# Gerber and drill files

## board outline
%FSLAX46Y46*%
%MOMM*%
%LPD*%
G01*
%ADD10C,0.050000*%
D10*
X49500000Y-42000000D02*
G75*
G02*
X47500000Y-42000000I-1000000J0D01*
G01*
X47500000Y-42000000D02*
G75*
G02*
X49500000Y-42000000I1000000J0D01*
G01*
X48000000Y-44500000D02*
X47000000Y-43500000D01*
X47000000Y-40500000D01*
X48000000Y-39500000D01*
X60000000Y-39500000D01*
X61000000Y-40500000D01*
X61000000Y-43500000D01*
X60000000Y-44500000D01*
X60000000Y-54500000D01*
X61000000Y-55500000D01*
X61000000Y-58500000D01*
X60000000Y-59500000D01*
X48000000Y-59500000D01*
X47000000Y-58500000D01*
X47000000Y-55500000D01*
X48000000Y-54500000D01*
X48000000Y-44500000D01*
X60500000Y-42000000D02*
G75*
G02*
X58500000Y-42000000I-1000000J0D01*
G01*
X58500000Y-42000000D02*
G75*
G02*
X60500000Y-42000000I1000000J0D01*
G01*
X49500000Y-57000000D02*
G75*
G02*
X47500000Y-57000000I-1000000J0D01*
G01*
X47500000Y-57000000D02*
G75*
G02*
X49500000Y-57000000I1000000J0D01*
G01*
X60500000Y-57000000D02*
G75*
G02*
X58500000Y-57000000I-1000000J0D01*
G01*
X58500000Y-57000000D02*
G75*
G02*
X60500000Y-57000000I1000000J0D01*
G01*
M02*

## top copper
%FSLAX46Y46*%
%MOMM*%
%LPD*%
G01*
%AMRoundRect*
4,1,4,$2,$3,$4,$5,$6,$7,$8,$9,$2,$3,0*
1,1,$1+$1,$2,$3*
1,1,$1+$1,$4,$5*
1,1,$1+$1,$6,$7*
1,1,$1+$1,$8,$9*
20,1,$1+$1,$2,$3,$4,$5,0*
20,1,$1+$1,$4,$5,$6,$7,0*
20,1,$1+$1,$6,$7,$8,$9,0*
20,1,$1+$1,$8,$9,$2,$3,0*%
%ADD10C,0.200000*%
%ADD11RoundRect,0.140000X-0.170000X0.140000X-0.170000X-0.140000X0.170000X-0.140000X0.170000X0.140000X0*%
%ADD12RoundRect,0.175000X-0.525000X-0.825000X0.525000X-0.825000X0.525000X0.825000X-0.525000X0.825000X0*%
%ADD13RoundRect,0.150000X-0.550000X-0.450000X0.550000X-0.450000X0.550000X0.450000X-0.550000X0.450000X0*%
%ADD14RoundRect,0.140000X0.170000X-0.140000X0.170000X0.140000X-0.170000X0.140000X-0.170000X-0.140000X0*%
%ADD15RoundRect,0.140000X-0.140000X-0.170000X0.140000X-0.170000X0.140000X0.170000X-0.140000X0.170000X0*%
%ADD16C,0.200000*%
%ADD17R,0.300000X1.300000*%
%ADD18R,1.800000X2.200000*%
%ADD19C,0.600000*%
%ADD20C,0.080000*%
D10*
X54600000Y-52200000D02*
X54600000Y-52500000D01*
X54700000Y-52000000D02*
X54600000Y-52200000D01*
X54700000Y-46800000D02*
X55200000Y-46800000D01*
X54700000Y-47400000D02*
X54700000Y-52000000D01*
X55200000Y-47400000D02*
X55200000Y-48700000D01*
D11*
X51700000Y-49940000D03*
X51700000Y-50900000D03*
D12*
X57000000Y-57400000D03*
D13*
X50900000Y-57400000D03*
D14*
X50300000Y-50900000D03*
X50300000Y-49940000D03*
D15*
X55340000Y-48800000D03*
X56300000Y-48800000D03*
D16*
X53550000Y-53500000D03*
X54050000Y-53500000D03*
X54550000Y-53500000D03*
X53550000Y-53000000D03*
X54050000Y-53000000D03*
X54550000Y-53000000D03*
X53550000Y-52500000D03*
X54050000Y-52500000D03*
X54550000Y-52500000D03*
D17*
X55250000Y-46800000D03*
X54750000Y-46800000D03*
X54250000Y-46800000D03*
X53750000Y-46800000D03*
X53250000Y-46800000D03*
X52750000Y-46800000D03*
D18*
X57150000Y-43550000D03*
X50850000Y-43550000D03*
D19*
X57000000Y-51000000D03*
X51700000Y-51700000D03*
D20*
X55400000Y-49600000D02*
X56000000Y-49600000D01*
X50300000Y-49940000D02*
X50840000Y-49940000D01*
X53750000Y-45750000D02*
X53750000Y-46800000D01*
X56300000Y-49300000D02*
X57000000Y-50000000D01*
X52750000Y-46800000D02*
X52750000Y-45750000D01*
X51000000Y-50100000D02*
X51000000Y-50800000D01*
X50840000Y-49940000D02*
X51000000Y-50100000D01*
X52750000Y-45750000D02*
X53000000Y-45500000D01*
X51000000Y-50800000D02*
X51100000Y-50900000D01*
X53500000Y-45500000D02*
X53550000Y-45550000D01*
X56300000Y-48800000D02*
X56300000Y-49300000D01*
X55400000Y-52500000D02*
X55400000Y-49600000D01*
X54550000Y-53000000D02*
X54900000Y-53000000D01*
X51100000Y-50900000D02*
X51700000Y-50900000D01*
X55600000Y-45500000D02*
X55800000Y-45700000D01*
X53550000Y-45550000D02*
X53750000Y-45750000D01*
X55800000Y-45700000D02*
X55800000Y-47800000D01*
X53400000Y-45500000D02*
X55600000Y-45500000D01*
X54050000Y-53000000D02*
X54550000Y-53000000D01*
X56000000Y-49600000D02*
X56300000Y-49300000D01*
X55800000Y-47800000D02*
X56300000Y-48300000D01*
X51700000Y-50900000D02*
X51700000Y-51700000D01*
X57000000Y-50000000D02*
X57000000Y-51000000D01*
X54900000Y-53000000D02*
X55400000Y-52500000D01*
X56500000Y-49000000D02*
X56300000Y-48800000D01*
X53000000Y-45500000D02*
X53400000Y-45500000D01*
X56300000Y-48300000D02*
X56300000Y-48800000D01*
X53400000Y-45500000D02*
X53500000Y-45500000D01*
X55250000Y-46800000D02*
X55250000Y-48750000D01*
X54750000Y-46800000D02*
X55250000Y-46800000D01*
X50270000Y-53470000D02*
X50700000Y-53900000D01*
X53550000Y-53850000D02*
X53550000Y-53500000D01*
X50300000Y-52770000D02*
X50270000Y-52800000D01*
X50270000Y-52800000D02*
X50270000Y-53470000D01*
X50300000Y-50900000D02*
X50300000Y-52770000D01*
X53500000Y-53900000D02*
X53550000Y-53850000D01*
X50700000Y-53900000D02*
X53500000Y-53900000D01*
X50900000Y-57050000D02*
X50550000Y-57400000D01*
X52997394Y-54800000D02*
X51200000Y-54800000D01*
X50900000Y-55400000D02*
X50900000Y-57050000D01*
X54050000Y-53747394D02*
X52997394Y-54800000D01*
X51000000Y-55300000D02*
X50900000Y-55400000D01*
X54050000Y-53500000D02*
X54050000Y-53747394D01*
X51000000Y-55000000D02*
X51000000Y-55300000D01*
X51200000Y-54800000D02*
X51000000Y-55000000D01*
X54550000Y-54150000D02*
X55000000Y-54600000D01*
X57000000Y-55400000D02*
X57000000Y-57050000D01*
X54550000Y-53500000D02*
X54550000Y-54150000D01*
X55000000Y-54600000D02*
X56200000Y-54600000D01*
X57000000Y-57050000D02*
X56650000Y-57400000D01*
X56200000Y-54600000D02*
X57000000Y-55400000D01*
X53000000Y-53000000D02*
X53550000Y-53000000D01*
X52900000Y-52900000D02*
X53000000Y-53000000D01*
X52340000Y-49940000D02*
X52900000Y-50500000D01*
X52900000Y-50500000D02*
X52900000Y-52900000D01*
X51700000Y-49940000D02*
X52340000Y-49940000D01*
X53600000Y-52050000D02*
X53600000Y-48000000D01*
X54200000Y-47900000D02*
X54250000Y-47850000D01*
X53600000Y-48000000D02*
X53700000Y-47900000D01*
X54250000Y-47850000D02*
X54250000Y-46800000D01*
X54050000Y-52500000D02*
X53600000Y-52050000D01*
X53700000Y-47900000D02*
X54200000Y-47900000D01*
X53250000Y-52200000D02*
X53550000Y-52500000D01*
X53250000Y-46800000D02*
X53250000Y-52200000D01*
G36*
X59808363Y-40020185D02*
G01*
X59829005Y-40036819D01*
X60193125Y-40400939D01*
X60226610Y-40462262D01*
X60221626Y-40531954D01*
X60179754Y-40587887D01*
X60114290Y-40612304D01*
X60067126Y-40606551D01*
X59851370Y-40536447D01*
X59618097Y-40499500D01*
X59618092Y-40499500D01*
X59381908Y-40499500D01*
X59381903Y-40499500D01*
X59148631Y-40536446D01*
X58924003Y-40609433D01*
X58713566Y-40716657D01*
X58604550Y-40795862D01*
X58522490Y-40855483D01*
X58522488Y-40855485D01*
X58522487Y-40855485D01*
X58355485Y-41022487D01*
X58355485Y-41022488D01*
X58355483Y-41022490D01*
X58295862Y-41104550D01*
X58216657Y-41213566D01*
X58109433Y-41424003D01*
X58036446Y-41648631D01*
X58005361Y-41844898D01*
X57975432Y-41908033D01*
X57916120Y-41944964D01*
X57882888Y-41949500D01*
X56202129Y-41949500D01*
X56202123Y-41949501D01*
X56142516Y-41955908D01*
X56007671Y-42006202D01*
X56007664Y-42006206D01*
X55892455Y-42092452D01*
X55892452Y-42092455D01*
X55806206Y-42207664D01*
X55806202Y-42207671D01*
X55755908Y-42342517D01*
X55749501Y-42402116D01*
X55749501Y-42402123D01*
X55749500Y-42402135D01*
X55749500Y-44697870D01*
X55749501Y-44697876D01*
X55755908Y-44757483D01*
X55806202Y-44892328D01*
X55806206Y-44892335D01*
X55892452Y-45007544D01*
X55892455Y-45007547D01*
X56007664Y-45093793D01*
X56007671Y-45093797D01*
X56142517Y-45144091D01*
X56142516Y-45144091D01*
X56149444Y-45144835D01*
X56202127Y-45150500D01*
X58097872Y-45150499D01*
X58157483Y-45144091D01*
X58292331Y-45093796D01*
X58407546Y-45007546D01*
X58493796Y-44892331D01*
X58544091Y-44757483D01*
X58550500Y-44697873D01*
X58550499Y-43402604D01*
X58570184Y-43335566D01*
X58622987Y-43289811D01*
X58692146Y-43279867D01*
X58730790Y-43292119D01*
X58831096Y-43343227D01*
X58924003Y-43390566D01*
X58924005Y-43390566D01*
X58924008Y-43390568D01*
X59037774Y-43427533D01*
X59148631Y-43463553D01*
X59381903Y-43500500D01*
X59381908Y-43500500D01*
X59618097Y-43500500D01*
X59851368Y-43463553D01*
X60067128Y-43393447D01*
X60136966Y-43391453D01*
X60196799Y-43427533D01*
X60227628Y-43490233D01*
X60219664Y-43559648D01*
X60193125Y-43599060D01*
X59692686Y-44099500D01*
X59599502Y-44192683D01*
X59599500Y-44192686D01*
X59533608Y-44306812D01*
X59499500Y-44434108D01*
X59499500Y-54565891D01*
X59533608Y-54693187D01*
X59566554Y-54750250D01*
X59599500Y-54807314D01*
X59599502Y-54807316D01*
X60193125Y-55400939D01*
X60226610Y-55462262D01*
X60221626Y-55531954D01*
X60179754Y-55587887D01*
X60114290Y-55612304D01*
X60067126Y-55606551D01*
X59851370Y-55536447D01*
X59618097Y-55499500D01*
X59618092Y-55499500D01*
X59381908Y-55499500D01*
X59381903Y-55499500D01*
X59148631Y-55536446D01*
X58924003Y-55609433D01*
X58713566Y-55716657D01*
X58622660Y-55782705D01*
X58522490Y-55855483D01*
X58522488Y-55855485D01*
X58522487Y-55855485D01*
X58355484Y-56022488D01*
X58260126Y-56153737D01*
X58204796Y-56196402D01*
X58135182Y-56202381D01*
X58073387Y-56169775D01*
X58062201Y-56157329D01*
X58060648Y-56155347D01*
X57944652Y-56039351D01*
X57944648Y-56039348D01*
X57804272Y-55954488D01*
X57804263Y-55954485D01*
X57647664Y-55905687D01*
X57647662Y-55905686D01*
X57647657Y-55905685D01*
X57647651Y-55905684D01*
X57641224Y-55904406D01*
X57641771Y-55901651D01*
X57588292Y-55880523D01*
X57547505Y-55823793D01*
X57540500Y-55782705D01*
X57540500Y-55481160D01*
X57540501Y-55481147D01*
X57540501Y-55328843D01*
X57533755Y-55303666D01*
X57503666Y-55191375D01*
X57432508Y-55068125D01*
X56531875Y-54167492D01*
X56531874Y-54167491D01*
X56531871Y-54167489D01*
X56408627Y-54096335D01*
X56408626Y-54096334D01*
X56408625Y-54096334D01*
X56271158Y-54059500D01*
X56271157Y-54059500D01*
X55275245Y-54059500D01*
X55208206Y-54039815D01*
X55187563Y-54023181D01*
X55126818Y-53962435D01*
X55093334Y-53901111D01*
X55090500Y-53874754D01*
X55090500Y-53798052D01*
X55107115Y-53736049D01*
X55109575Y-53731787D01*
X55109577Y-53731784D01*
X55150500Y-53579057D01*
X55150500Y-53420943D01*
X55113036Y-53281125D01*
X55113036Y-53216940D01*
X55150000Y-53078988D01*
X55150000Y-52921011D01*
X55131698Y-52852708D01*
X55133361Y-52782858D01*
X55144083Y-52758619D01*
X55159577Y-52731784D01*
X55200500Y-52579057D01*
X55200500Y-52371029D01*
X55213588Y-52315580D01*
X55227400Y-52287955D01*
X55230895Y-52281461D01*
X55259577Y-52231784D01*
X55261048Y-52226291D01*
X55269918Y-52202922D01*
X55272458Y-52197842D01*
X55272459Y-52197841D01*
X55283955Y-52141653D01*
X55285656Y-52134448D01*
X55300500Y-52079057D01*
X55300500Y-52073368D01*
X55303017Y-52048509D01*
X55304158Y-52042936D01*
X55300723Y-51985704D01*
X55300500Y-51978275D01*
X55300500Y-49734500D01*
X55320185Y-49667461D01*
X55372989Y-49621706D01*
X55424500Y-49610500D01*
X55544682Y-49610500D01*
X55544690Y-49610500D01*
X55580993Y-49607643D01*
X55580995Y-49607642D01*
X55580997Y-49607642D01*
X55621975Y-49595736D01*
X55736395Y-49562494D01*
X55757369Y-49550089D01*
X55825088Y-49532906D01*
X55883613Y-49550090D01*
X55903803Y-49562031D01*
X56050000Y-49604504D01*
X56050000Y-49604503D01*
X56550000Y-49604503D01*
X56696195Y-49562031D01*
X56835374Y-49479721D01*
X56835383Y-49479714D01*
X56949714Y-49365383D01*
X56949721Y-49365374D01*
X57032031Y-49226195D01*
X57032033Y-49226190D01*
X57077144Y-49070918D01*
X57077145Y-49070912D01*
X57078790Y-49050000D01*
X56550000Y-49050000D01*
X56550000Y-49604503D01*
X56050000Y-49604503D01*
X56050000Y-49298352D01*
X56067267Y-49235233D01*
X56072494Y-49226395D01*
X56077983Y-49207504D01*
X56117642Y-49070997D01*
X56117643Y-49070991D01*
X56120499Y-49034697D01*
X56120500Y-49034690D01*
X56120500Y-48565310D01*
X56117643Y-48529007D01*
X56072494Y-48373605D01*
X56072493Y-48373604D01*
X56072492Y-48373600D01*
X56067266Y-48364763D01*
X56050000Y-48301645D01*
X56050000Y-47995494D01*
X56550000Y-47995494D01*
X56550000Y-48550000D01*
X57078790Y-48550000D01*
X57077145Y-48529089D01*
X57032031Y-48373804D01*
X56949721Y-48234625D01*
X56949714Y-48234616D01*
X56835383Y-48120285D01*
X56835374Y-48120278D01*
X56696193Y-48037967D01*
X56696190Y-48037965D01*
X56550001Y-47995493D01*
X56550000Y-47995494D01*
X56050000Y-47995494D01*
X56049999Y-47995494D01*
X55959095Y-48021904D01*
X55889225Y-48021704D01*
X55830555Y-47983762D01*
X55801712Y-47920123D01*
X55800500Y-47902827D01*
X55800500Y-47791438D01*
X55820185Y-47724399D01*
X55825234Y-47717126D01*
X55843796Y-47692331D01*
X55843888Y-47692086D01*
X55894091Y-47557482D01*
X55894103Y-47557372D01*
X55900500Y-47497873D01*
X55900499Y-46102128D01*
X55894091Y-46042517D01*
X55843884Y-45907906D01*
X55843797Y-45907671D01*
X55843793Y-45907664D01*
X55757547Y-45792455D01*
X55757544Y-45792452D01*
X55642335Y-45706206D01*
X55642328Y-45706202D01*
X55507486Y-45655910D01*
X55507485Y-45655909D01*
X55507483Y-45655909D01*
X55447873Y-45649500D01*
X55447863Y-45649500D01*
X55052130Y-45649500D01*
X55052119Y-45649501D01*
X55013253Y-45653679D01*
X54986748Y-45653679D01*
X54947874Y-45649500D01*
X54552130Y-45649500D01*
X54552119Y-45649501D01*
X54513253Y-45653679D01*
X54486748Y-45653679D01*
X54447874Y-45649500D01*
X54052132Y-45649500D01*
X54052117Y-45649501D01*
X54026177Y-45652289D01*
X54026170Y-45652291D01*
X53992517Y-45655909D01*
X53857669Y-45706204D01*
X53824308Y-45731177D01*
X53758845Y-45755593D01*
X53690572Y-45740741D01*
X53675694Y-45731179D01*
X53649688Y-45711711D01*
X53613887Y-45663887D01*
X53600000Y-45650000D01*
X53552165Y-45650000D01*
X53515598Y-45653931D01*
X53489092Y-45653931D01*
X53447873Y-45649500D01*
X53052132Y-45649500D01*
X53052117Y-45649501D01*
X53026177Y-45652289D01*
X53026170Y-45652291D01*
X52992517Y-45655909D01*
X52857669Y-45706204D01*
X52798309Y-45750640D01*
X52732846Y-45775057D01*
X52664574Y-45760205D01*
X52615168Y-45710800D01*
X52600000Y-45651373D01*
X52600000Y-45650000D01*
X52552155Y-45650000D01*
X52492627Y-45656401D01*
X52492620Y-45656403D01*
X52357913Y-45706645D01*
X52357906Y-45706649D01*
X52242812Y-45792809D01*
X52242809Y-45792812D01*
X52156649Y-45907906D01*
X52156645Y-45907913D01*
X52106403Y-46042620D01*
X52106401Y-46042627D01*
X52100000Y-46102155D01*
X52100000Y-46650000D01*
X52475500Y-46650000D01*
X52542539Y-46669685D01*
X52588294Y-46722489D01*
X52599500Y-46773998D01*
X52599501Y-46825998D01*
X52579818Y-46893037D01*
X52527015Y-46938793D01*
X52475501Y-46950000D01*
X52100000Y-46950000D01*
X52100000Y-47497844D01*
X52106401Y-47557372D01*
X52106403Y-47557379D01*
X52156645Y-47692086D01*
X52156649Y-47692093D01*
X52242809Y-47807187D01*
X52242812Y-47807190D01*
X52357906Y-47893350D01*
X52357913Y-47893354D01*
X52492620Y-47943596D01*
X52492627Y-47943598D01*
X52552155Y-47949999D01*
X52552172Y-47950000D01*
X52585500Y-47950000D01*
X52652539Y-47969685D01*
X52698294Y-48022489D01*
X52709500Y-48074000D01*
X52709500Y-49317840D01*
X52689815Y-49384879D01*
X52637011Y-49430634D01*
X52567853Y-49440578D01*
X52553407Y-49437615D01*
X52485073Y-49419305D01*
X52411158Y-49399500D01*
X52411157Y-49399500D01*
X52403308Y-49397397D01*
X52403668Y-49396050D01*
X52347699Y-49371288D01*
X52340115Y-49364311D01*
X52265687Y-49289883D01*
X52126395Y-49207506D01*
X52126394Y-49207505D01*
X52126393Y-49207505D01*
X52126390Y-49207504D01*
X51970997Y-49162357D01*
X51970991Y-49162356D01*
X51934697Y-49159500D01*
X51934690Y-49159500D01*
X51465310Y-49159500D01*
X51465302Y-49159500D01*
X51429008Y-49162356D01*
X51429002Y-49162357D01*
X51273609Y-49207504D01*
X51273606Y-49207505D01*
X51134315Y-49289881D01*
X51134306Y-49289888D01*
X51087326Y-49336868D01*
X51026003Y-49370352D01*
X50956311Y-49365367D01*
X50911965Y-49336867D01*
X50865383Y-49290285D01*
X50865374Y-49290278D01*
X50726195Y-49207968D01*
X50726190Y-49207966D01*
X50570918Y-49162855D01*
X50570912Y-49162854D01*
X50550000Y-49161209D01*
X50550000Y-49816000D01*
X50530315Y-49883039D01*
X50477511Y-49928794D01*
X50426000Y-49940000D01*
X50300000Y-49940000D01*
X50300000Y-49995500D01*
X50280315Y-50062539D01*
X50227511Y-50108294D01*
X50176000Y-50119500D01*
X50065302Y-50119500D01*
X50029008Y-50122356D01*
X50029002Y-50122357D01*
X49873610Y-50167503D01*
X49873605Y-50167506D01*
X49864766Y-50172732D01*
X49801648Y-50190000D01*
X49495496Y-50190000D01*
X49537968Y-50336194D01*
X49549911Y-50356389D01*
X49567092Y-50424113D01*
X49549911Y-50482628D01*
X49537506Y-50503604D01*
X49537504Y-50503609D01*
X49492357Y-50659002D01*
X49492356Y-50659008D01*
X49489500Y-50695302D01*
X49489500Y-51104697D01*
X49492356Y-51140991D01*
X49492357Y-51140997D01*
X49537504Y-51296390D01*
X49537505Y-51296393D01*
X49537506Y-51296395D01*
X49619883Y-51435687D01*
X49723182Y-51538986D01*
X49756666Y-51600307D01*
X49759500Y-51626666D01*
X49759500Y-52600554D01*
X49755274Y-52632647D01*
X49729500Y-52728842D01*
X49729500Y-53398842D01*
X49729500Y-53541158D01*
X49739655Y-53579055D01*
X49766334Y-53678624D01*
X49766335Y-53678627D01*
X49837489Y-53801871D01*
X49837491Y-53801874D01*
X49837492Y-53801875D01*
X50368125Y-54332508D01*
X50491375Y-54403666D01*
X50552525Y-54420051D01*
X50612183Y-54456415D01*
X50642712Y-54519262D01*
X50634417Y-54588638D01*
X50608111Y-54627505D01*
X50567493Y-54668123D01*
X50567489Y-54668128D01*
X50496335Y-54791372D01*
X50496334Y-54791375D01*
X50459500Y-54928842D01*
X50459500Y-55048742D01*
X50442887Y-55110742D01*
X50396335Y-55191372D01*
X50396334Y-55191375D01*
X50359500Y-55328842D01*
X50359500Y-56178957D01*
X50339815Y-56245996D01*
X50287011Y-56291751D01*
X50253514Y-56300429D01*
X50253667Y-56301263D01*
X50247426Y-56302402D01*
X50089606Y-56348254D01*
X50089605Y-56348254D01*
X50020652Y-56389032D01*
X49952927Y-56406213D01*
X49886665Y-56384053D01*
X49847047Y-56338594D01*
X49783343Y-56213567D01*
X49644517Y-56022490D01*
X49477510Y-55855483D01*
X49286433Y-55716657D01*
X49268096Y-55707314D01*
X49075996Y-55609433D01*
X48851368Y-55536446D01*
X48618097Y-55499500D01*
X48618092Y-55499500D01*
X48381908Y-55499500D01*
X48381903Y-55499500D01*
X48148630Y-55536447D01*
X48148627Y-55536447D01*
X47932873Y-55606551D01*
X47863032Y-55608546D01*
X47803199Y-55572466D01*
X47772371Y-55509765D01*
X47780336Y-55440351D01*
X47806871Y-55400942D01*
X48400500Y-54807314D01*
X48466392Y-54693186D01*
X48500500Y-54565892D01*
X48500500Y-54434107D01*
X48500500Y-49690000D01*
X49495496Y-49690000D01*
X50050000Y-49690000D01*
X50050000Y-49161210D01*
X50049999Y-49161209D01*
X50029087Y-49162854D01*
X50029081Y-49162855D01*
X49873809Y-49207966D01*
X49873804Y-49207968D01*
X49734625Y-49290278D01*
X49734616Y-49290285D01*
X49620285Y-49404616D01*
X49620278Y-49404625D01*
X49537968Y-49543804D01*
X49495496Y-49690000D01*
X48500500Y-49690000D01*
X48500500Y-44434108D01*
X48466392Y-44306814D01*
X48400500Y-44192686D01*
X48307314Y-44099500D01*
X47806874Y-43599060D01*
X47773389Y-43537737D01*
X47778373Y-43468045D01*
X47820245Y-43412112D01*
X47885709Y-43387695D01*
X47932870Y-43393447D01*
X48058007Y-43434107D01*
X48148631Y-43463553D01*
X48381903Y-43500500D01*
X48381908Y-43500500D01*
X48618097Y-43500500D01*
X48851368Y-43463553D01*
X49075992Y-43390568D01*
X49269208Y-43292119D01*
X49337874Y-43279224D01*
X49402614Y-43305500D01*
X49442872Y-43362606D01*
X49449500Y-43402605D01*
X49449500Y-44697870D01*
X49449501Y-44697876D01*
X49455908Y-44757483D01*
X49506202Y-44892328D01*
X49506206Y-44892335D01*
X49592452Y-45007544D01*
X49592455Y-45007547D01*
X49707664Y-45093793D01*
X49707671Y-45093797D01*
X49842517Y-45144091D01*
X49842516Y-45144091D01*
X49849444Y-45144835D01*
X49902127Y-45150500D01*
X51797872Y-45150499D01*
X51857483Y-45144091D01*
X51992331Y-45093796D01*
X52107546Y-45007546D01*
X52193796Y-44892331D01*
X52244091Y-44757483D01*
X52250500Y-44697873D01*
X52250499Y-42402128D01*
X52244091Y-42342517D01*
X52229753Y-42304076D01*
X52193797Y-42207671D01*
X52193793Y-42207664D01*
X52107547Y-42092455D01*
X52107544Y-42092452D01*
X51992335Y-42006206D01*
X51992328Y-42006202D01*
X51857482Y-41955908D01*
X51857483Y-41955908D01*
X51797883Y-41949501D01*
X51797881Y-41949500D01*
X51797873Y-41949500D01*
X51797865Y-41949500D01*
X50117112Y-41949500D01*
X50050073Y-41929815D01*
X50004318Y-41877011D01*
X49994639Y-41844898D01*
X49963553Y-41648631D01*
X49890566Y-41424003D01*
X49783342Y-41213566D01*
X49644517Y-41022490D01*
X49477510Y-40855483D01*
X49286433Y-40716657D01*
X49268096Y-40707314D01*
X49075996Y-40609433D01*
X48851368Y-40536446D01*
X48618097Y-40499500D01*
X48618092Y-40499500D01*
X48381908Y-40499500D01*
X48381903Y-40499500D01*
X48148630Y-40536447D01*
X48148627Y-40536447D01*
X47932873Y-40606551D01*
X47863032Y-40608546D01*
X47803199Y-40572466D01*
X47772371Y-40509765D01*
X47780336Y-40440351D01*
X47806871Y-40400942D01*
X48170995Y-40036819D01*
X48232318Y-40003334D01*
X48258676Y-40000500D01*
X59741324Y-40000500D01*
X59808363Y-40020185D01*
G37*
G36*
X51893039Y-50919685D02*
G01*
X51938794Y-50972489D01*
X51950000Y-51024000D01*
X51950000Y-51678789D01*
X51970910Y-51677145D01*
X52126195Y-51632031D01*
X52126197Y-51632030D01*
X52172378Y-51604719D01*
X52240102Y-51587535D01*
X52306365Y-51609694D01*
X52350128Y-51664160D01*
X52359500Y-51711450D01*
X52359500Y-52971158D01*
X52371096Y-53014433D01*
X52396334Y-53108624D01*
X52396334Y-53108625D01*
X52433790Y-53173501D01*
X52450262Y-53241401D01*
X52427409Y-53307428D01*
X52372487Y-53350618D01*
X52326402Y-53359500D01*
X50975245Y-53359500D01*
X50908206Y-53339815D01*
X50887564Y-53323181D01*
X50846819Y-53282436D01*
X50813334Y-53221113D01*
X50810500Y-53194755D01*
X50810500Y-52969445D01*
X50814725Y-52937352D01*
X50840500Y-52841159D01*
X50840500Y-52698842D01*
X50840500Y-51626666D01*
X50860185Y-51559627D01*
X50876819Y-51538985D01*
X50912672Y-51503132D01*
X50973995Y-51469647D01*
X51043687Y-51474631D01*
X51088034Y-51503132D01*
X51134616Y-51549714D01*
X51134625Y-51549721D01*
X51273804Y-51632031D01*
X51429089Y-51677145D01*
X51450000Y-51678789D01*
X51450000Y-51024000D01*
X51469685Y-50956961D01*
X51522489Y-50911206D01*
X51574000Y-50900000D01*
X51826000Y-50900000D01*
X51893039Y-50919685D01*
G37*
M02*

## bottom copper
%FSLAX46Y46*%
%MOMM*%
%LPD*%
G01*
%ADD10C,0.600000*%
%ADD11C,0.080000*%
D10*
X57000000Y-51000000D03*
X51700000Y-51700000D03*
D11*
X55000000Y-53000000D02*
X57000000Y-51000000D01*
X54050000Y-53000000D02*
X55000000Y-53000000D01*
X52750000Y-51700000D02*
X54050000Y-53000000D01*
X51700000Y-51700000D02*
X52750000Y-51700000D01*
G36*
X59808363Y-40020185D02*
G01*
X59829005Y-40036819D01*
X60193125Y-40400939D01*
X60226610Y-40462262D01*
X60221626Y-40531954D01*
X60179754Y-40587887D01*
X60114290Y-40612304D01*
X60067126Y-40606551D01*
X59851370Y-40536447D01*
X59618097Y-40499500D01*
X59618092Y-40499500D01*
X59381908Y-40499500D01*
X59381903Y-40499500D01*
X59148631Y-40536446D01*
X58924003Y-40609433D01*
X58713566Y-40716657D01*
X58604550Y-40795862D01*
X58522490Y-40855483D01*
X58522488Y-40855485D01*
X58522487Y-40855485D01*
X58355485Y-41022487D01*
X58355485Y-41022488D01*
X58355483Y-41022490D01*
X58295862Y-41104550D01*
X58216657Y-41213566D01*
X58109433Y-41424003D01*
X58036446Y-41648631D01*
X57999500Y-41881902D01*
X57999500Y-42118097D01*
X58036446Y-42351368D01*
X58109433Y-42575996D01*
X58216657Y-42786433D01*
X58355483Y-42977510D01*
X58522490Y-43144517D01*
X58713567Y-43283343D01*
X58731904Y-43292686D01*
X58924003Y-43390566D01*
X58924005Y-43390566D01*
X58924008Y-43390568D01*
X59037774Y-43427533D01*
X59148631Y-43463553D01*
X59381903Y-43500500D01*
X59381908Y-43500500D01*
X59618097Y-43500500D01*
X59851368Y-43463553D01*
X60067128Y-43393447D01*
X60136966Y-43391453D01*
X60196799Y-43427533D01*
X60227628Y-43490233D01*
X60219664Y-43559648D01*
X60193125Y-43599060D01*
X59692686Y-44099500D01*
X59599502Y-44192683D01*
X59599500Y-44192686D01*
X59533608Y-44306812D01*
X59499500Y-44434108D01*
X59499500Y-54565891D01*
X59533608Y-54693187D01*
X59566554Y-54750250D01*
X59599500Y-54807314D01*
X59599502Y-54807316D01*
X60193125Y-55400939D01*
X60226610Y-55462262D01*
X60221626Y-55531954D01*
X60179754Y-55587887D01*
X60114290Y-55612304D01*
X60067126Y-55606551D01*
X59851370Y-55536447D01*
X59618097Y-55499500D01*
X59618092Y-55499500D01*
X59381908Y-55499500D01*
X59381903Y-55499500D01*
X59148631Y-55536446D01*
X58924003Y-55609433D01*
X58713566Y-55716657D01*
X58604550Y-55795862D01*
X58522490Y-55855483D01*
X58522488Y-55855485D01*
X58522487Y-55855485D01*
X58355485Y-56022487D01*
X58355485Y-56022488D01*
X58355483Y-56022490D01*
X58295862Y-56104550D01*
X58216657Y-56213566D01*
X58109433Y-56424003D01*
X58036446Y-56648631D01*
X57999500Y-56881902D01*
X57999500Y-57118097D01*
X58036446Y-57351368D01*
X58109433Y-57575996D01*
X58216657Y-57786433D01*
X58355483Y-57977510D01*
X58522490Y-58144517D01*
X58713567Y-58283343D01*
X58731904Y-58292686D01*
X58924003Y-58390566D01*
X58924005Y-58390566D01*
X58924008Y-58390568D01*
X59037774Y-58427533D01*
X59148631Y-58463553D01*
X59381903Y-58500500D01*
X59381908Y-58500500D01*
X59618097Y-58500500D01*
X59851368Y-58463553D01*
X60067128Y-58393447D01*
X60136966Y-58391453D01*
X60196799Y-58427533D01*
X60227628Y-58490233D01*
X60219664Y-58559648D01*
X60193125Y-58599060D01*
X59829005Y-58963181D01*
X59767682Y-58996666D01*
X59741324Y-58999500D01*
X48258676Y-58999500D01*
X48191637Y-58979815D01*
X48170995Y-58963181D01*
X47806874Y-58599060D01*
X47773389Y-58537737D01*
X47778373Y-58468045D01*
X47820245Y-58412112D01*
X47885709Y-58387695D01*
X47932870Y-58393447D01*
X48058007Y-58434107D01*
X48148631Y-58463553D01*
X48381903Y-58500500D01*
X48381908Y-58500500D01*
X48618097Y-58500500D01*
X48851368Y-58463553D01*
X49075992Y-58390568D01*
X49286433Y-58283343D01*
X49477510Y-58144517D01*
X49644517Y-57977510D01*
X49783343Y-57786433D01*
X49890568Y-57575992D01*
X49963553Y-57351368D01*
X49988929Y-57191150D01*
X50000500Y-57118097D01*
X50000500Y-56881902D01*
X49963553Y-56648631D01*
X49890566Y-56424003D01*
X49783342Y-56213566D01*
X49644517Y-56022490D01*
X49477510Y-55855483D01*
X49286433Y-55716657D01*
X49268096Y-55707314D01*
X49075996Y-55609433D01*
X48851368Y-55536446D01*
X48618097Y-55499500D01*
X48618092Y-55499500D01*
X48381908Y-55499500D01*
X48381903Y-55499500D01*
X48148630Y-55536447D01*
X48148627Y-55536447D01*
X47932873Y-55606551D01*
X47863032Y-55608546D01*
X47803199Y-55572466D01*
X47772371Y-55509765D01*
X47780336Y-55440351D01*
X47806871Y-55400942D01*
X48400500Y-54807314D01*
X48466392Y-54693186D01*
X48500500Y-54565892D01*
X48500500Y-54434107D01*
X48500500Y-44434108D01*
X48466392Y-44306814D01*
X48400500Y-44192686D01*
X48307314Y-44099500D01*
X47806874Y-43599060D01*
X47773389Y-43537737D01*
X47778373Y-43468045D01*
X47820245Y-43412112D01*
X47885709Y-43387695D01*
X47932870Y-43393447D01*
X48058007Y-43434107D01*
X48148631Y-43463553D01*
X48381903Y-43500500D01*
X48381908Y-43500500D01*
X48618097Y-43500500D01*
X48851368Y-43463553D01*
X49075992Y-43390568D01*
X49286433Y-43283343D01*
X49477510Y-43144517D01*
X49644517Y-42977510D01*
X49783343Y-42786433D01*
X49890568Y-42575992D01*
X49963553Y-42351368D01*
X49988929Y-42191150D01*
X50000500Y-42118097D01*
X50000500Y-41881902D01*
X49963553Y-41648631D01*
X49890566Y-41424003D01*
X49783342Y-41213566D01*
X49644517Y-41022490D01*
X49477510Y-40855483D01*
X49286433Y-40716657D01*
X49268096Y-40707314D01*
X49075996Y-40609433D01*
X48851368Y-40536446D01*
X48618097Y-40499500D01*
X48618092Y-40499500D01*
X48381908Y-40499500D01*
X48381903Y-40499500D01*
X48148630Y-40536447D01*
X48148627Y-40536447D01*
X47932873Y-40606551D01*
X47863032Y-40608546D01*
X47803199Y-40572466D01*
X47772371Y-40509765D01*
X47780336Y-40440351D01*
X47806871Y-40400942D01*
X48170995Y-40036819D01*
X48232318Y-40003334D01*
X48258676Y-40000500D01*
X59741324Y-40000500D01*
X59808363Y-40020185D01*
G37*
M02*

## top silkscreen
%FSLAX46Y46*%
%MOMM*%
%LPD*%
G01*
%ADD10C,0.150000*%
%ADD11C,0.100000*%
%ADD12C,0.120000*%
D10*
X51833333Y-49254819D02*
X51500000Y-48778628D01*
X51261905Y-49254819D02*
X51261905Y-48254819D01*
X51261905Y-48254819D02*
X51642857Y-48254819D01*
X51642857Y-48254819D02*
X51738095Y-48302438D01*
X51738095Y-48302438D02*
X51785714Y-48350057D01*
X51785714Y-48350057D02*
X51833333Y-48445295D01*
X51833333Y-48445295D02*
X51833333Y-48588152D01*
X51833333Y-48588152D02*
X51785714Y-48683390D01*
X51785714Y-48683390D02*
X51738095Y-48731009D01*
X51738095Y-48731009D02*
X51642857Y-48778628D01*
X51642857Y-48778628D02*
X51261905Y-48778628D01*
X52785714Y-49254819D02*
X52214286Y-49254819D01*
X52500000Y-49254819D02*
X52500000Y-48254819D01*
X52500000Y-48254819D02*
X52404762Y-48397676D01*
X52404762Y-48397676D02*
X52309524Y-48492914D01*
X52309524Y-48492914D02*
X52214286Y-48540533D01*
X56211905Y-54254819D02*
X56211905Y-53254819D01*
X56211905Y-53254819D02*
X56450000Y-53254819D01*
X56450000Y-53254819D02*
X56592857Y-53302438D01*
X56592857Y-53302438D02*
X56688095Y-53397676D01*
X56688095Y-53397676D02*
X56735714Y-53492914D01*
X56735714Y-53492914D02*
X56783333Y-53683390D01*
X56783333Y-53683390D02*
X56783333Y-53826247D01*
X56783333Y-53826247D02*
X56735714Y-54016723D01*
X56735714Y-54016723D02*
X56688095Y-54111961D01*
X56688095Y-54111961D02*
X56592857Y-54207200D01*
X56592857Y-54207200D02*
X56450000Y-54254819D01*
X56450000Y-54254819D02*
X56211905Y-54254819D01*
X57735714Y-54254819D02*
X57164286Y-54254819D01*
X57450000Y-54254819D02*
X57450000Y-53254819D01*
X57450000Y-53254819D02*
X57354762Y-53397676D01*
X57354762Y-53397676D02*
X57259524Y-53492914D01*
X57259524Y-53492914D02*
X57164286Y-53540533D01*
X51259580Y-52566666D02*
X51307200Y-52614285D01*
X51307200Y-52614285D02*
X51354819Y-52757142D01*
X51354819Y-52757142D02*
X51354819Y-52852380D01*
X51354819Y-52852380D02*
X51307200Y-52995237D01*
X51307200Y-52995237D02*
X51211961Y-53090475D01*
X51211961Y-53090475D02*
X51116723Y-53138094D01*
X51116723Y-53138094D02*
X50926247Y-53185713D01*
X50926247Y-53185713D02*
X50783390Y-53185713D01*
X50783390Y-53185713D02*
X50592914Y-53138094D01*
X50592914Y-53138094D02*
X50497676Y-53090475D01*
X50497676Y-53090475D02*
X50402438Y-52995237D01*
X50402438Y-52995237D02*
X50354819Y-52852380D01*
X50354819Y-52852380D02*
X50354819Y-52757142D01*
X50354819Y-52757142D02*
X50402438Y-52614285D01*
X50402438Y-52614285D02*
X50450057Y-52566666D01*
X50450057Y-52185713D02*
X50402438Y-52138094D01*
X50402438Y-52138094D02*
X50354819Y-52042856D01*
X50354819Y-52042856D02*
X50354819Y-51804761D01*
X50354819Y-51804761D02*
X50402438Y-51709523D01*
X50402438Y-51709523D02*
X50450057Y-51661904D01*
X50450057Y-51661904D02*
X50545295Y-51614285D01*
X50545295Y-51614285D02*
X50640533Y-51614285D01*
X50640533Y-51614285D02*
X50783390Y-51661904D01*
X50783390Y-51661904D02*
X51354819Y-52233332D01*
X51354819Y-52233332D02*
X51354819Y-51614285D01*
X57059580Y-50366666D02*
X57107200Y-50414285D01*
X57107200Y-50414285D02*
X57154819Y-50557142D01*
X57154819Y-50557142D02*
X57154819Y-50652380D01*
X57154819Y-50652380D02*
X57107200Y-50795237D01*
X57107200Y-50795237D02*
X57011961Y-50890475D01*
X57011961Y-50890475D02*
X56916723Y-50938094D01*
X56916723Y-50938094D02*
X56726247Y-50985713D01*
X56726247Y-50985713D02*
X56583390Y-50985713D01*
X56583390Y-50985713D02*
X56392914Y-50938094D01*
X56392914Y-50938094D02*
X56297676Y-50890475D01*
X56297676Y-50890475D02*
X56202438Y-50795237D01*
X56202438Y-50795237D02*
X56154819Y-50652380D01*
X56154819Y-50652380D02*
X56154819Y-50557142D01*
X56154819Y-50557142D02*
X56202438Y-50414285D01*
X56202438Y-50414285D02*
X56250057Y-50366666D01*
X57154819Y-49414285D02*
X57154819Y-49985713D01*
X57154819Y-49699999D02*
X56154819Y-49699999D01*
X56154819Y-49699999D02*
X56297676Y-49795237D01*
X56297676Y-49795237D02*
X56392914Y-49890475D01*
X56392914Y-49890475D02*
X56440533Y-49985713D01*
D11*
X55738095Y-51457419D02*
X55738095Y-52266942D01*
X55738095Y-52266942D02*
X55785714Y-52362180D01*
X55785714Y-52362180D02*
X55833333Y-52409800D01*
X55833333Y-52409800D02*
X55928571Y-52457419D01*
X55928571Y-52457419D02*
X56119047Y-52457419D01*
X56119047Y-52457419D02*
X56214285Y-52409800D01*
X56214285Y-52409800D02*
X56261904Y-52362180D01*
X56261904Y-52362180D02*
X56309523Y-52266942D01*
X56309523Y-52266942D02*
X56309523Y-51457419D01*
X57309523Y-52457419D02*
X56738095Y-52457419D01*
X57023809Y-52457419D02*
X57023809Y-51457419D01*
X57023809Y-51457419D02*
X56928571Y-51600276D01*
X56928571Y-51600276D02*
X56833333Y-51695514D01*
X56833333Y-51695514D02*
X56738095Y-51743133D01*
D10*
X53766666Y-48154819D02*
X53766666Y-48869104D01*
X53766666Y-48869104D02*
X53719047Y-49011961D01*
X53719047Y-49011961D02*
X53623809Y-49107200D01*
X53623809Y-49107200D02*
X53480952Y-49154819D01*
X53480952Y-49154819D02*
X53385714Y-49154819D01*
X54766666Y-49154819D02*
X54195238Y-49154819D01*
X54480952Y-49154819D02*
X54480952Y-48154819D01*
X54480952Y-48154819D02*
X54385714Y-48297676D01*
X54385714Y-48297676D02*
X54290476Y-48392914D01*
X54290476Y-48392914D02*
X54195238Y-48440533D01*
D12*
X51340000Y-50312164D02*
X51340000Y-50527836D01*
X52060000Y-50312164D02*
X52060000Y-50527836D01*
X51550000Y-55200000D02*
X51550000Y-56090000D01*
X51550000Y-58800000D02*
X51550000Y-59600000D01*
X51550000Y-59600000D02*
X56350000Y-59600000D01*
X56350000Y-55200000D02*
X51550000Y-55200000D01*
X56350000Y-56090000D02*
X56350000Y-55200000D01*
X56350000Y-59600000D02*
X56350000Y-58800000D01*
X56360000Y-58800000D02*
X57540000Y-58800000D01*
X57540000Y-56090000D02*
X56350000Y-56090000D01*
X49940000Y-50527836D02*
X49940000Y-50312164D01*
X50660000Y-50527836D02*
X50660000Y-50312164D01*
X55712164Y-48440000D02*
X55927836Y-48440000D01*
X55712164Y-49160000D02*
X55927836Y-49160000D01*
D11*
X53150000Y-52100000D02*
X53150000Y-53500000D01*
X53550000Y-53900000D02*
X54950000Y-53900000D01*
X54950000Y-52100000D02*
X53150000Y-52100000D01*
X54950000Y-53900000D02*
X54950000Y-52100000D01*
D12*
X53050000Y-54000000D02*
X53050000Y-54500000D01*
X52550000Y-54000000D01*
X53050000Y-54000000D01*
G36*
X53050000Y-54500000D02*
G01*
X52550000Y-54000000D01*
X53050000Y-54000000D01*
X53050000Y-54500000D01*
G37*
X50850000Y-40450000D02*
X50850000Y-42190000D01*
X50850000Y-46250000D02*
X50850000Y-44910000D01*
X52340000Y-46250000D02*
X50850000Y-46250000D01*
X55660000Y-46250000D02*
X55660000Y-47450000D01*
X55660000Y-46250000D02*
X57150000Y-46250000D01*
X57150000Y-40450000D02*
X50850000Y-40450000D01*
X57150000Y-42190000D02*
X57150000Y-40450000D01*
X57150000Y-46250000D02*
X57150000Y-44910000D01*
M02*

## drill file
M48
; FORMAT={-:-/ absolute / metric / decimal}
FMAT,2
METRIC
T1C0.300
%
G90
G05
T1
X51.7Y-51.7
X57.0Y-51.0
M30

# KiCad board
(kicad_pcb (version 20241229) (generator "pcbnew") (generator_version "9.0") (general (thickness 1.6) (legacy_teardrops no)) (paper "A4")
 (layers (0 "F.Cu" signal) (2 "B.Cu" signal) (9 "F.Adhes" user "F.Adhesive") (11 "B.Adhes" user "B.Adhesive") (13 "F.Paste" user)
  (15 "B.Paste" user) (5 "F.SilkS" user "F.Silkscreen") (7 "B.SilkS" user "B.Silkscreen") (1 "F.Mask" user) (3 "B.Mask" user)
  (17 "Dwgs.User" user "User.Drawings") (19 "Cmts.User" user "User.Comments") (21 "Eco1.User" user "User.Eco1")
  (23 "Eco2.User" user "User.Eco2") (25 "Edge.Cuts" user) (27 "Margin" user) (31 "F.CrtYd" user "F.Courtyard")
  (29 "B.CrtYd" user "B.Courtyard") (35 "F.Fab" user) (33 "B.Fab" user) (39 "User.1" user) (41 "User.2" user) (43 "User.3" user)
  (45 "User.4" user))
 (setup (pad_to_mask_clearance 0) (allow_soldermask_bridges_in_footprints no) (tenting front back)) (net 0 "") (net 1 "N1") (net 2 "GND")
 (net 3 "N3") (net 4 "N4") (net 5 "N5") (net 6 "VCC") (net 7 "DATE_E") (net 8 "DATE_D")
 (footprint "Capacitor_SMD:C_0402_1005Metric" (layer "F.Cu") (at 51.7 50.42 -90)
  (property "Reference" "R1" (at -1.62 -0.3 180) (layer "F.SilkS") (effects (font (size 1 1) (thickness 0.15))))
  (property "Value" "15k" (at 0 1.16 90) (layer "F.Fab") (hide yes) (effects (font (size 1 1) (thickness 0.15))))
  (fp_line (start -0.107836 0.36) (end 0.107836 0.36) (stroke (width 0.12) (type solid)) (layer "F.SilkS"))
  (fp_line (start -0.107836 -0.36) (end 0.107836 -0.36) (stroke (width 0.12) (type solid)) (layer "F.SilkS"))
  (pad "1" smd roundrect (at -0.48 0 270) (size 0.56 0.62) (layers "F.Cu" "F.Mask" "F.Paste") (roundrect_rratio 0.25) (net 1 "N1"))
  (pad "2" smd roundrect (at 0.48 0 270) (size 0.56 0.62) (layers "F.Cu" "F.Mask" "F.Paste") (roundrect_rratio 0.25) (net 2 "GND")))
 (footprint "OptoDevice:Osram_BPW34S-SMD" (layer "F.Cu") (at 53.95 57.4 180)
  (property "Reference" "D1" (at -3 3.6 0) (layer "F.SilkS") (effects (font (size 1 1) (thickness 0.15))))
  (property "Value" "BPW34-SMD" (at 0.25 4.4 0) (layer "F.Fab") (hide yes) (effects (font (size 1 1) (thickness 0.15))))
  (fp_line (start 2.4 2.2) (end 2.4 1.31) (stroke (width 0.12) (type solid)) (layer "F.SilkS"))
  (fp_line (start 2.4 -1.4) (end 2.4 -2.2) (stroke (width 0.12) (type solid)) (layer "F.SilkS"))
  (fp_line (start 2.4 -2.2) (end -2.4 -2.2) (stroke (width 0.12) (type solid)) (layer "F.SilkS"))
  (fp_line (start -2.4 2.2) (end 2.4 2.2) (stroke (width 0.12) (type solid)) (layer "F.SilkS"))
  (fp_line (start -2.4 1.31) (end -2.4 2.2) (stroke (width 0.12) (type solid)) (layer "F.SilkS"))
  (fp_line (start -2.4 -2.2) (end -2.4 -1.4) (stroke (width 0.12) (type solid)) (layer "F.SilkS"))
  (fp_line (start -2.41 -1.4) (end -3.59 -1.4) (stroke (width 0.12) (type solid)) (layer "F.SilkS"))
  (fp_line (start -3.59 1.31) (end -2.4 1.31) (stroke (width 0.12) (type solid)) (layer "F.SilkS"))
  (pad "" smd roundrect (at -3.05 0) (size 1.3 1.9) (layers "F.Paste") (roundrect_rratio 0.125))
  (pad "" smd roundrect (at -3.05 0) (size 1.5 2.1) (layers "F.Mask") (roundrect_rratio 0.125))
  (pad "" smd roundrect (at 3.05 0) (size 1.3 1.1) (layers "F.Paste") (roundrect_rratio 0.125))
  (pad "" smd roundrect (at 3.05 0) (size 1.5 1.3) (layers "F.Mask") (roundrect_rratio 0.125))
  (pad "1" smd roundrect (at -3.05 0) (size 1.4 2) (layers "F.Cu" "F.Mask") (roundrect_rratio 0.125) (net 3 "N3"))
  (pad "2" smd roundrect (at 3.05 0) (size 1.4 1.2) (layers "F.Cu" "F.Mask") (roundrect_rratio 0.125) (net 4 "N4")))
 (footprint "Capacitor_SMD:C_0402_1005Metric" (layer "F.Cu") (at 50.3 50.42 90)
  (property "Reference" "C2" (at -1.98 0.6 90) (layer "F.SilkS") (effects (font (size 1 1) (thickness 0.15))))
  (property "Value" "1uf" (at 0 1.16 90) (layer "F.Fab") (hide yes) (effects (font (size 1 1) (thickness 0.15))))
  (fp_line (start -0.107836 -0.36) (end 0.107836 -0.36) (stroke (width 0.12) (type solid)) (layer "F.SilkS"))
  (fp_line (start -0.107836 0.36) (end 0.107836 0.36) (stroke (width 0.12) (type solid)) (layer "F.SilkS"))
  (pad "1" smd roundrect (at -0.48 0 90) (size 0.56 0.62) (layers "F.Cu" "F.Mask" "F.Paste") (roundrect_rratio 0.25) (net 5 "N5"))
  (pad "2" smd roundrect (at 0.48 0 90) (size 0.56 0.62) (layers "F.Cu" "F.Mask" "F.Paste") (roundrect_rratio 0.25) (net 2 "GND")))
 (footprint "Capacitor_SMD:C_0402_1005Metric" (layer "F.Cu") (at 55.82 48.8)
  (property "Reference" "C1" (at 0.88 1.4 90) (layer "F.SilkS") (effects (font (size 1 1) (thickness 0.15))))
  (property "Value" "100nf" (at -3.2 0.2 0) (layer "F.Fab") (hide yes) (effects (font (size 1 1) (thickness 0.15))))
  (fp_line (start -0.107836 -0.36) (end 0.107836 -0.36) (stroke (width 0.12) (type solid)) (layer "F.SilkS"))
  (fp_line (start -0.107836 0.36) (end 0.107836 0.36) (stroke (width 0.12) (type solid)) (layer "F.SilkS"))
  (pad "1" smd roundrect (at -0.48 0) (size 0.56 0.62) (layers "F.Cu" "F.Mask" "F.Paste") (roundrect_rratio 0.25) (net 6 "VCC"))
  (pad "2" smd roundrect (at 0.48 0) (size 0.56 0.62) (layers "F.Cu" "F.Mask" "F.Paste") (roundrect_rratio 0.25) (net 2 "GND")))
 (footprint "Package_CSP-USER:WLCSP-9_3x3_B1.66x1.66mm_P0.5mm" (layer "F.Cu") (at 54.05 53)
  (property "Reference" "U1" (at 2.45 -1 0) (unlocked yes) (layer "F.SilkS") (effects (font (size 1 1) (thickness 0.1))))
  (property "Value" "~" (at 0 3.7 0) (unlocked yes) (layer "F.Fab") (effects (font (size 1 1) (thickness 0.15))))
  (fp_line (start -0.9 -0.9) (end -0.9 0.5) (stroke (width 0.1) (type default)) (layer "F.SilkS"))
  (fp_line (start -0.5 0.9) (end 0.9 0.9) (stroke (width 0.1) (type default)) (layer "F.SilkS"))
  (fp_line (start 0.9 -0.9) (end -0.9 -0.9) (stroke (width 0.1) (type default)) (layer "F.SilkS"))
  (fp_line (start 0.9 0.9) (end 0.9 -0.9) (stroke (width 0.1) (type default)) (layer "F.SilkS"))
  (fp_poly (pts (xy -1 1) (xy -1 1.5) (xy -1.5 1) (xy -1 1)) (stroke (width 0.12) (type solid)) (fill yes) (layer "F.SilkS"))
  (pad "1" smd circle (at -0.5 0.5) (size 0.2 0.2) (layers "F.Cu" "F.Paste") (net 5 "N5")
   (padstack (mode custom) (layer "B.Cu" (shape circle) (size 0.25 0.25) (zone_connect -1))))
  (pad "2" smd circle (at 0 0.5) (size 0.2 0.2) (layers "F.Cu" "F.Paste") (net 4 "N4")
   (padstack (mode custom) (layer "B.Cu" (shape circle) (size 0.25 0.25) (zone_connect -1))))
  (pad "3" smd circle (at 0.5 0.5) (size 0.2 0.2) (layers "F.Cu" "F.Paste") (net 3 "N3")
   (padstack (mode custom) (layer "B.Cu" (shape circle) (size 0.25 0.25) (zone_connect -1))))
  (pad "4" smd circle (at -0.5 0) (size 0.2 0.2) (layers "F.Cu" "F.Paste") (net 1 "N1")
   (padstack (mode custom) (layer "B.Cu" (shape circle) (size 0.25 0.25) (zone_connect -1))))
  (pad "5" smd circle (at 0 0) (size 0.2 0.2) (layers "F.Cu" "F.Paste") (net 2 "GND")
   (padstack (mode custom) (layer "B.Cu" (shape circle) (size 0.25 0.25) (zone_connect -1))))
  (pad "6" smd circle (at 0.5 0) (size 0.2 0.2) (layers "F.Cu" "F.Paste") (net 2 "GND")
   (padstack (mode custom) (layer "B.Cu" (shape circle) (size 0.25 0.25) (zone_connect -1))))
  (pad "7" smd circle (at -0.5 -0.5) (size 0.2 0.2) (layers "F.Cu" "F.Paste") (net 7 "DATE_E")
   (padstack (mode custom) (layer "B.Cu" (shape circle) (size 0.25 0.25) (zone_connect -1))))
  (pad "8" smd circle (at 0 -0.5) (size 0.2 0.2) (layers "F.Cu" "F.Paste") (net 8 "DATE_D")
   (padstack (mode custom) (layer "B.Cu" (shape circle) (size 0.25 0.25) (zone_connect -1))))
  (pad "9" smd circle (at 0.5 -0.5) (size 0.2 0.2) (layers "F.Cu" "F.Paste") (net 6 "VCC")
   (padstack (mode custom) (layer "B.Cu" (shape circle) (size 0.25 0.25) (zone_connect -1)))))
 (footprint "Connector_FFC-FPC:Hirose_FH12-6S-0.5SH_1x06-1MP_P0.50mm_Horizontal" (layer "F.Cu") (at 54 44.95 180)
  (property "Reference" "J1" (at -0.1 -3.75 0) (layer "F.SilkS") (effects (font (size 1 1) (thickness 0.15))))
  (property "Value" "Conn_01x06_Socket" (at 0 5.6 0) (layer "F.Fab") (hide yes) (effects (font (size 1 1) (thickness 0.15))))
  (fp_line (start 3.15 4.5) (end 3.15 2.76) (stroke (width 0.12) (type solid)) (layer "F.SilkS"))
  (fp_line (start 3.15 -1.3) (end 3.15 0.04) (stroke (width 0.12) (type solid)) (layer "F.SilkS"))
  (fp_line (start 1.66 -1.3) (end 3.15 -1.3) (stroke (width 0.12) (type solid)) (layer "F.SilkS"))
  (fp_line (start -1.66 -1.3) (end -1.66 -2.5) (stroke (width 0.12) (type solid)) (layer "F.SilkS"))
  (fp_line (start -1.66 -1.3) (end -3.15 -1.3) (stroke (width 0.12) (type solid)) (layer "F.SilkS"))
  (fp_line (start -3.15 4.5) (end 3.15 4.5) (stroke (width 0.12) (type solid)) (layer "F.SilkS"))
  (fp_line (start -3.15 2.76) (end -3.15 4.5) (stroke (width 0.12) (type solid)) (layer "F.SilkS"))
  (fp_line (start -3.15 -1.3) (end -3.15 0.04) (stroke (width 0.12) (type solid)) (layer "F.SilkS"))
  (pad "1" smd rect (at -1.25 -1.85 180) (size 0.3 1.3) (layers "F.Cu" "F.Mask" "F.Paste") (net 6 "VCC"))
  (pad "2" smd rect (at -0.75 -1.85 180) (size 0.3 1.3) (layers "F.Cu" "F.Mask" "F.Paste") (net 6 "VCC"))
  (pad "3" smd rect (at -0.25 -1.85 180) (size 0.3 1.3) (layers "F.Cu" "F.Mask" "F.Paste") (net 8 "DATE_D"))
  (pad "4" smd rect (at 0.25 -1.85 180) (size 0.3 1.3) (layers "F.Cu" "F.Mask" "F.Paste") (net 2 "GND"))
  (pad "5" smd rect (at 0.75 -1.85 180) (size 0.3 1.3) (layers "F.Cu" "F.Mask" "F.Paste") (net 7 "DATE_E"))
  (pad "6" smd rect (at 1.25 -1.85 180) (size 0.3 1.3) (layers "F.Cu" "F.Mask" "F.Paste") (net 2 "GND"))
  (pad "MP" smd rect (at -3.15 1.4 180) (size 1.8 2.2) (layers "F.Cu" "F.Mask" "F.Paste"))
  (pad "MP" smd rect (at 3.15 1.4 180) (size 1.8 2.2) (layers "F.Cu" "F.Mask" "F.Paste")))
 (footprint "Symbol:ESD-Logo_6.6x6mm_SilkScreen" (layer "B.Cu") (at 51.5 42.5 180)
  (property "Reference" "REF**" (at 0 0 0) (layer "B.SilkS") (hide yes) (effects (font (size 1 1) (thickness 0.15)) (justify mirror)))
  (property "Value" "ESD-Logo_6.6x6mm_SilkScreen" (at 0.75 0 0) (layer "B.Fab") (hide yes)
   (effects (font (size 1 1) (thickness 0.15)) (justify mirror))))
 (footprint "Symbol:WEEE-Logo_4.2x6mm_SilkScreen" (layer "B.Cu") (at 57 42.5 180)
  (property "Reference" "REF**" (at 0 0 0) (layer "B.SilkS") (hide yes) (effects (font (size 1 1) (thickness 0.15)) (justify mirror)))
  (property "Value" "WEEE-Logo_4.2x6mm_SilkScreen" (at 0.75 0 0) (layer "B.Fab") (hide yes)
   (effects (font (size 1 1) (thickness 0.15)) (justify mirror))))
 (gr_line (start 54.6 52.2) (end 54.6 52.5) (stroke (width 0.2) (type default)) (layer "F.Cu") (net 6))
 (gr_line (start 54.7 52) (end 54.6 52.2) (stroke (width 0.2) (type default)) (layer "F.Cu") (net 6))
 (gr_line (start 54.7 46.8) (end 55.2 46.8) (stroke (width 0.2) (type default)) (layer "F.Cu") (net 6))
 (gr_line (start 54.7 47.4) (end 54.7 52) (stroke (width 0.2) (type default)) (layer "F.Cu") (net 6))
 (gr_line (start 55.2 47.4) (end 55.2 48.7) (stroke (width 0.2) (type default)) (layer "F.Cu") (net 6))
 (gr_circle (center 48.5 42) (end 47.5 42) (stroke (width 0.05) (type default)) (fill no) (layer "Edge.Cuts"))
 (gr_poly
  (pts (xy 48 44.5) (xy 47 43.5) (xy 47 40.5) (xy 48 39.5) (xy 60 39.5) (xy 61 40.5) (xy 61 43.5) (xy 60 44.5) (xy 60 54.5) (xy 61 55.5)
   (xy 61 58.5) (xy 60 59.5) (xy 48 59.5) (xy 47 58.5) (xy 47 55.5) (xy 48 54.5))
  (stroke (width 0.05) (type solid)) (fill no) (layer "Edge.Cuts"))
 (gr_circle (center 59.5 42) (end 60.5 42) (stroke (width 0.05) (type default)) (fill no) (layer "Edge.Cuts"))
 (gr_circle (center 48.5 57) (end 49.5 57) (stroke (width 0.05) (type default)) (fill no) (layer "Edge.Cuts"))
 (gr_circle (center 59.5 57) (end 60.5 57) (stroke (width 0.05) (type default)) (fill no) (layer "Edge.Cuts"))
 (segment (start 55.4 49.6) (end 56 49.6) (width 0.08) (layer "F.Cu") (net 2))
 (segment (start 50.3 49.94) (end 50.84 49.94) (width 0.08) (layer "F.Cu") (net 2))
 (segment (start 53.75 45.75) (end 53.75 46.8) (width 0.08) (layer "F.Cu") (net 2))
 (segment (start 56.3 49.3) (end 57 50) (width 0.08) (layer "F.Cu") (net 2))
 (segment (start 52.75 46.8) (end 52.75 45.75) (width 0.08) (layer "F.Cu") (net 2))
 (segment (start 51 50.1) (end 51 50.8) (width 0.08) (layer "F.Cu") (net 2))
 (segment (start 50.84 49.94) (end 51 50.1) (width 0.08) (layer "F.Cu") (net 2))
 (segment (start 52.75 45.75) (end 53 45.5) (width 0.08) (layer "F.Cu") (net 2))
 (segment (start 51 50.8) (end 51.1 50.9) (width 0.08) (layer "F.Cu") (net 2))
 (segment (start 53.5 45.5) (end 53.55 45.55) (width 0.08) (layer "F.Cu") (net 2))
 (segment (start 56.3 48.8) (end 56.3 49.3) (width 0.08) (layer "F.Cu") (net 2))
 (segment (start 55.4 52.5) (end 55.4 49.6) (width 0.08) (layer "F.Cu") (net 2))
 (segment (start 54.55 53) (end 54.9 53) (width 0.08) (layer "F.Cu") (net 2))
 (segment (start 51.1 50.9) (end 51.7 50.9) (width 0.08) (layer "F.Cu") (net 2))
 (segment (start 55.6 45.5) (end 55.8 45.7) (width 0.08) (layer "F.Cu") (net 2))
 (segment (start 53.55 45.55) (end 53.75 45.75) (width 0.08) (layer "F.Cu") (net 2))
 (segment (start 55.8 45.7) (end 55.8 47.8) (width 0.08) (layer "F.Cu") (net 2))
 (segment (start 53.4 45.5) (end 55.6 45.5) (width 0.08) (layer "F.Cu") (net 2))
 (segment (start 54.05 53) (end 54.55 53) (width 0.08) (layer "F.Cu") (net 2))
 (segment (start 56 49.6) (end 56.3 49.3) (width 0.08) (layer "F.Cu") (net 2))
 (segment (start 55.8 47.8) (end 56.3 48.3) (width 0.08) (layer "F.Cu") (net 2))
 (segment (start 51.7 50.9) (end 51.7 51.7) (width 0.08) (layer "F.Cu") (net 2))
 (segment (start 57 50) (end 57 51) (width 0.08) (layer "F.Cu") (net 2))
 (segment (start 54.9 53) (end 55.4 52.5) (width 0.08) (layer "F.Cu") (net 2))
 (segment (start 56.5 49) (end 56.3 48.8) (width 0.08) (layer "F.Cu") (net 2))
 (segment (start 53 45.5) (end 53.4 45.5) (width 0.08) (layer "F.Cu") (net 2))
 (segment (start 56.3 48.3) (end 56.3 48.8) (width 0.08) (layer "F.Cu") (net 2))
 (segment (start 53.4 45.5) (end 53.5 45.5) (width 0.08) (layer "F.Cu") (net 2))
 (via (at 57 51) (size 0.6) (drill 0.3) (layers "F.Cu" "B.Cu") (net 2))
 (via (at 51.7 51.7) (size 0.6) (drill 0.3) (layers "F.Cu" "B.Cu") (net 2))
 (segment (start 55 53) (end 57 51) (width 0.08) (layer "B.Cu") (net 2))
 (segment (start 54.05 53) (end 55 53) (width 0.08) (layer "B.Cu") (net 2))
 (segment (start 52.75 51.7) (end 54.05 53) (width 0.08) (layer "B.Cu") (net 2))
 (segment (start 51.7 51.7) (end 52.75 51.7) (width 0.08) (layer "B.Cu") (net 2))
 (segment (start 55.25 46.8) (end 55.25 48.75) (width 0.08) (layer "F.Cu") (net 6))
 (segment (start 54.75 46.8) (end 55.25 46.8) (width 0.08) (layer "F.Cu") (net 6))
 (segment (start 50.27 53.47) (end 50.7 53.9) (width 0.08) (layer "F.Cu") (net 5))
 (segment (start 53.55 53.85) (end 53.55 53.5) (width 0.08) (layer "F.Cu") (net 5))
 (segment (start 50.3 52.77) (end 50.27 52.8) (width 0.08) (layer "F.Cu") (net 5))
 (segment (start 50.27 52.8) (end 50.27 53.47) (width 0.08) (layer "F.Cu") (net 5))
 (segment (start 50.3 50.9) (end 50.3 52.77) (width 0.08) (layer "F.Cu") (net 5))
 (segment (start 53.5 53.9) (end 53.55 53.85) (width 0.08) (layer "F.Cu") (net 5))
 (segment (start 50.7 53.9) (end 53.5 53.9) (width 0.08) (layer "F.Cu") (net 5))
 (segment (start 50.9 57.05) (end 50.55 57.4) (width 0.08) (layer "F.Cu") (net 4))
 (segment (start 52.997394 54.8) (end 51.2 54.8) (width 0.08) (layer "F.Cu") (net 4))
 (segment (start 50.9 55.4) (end 50.9 57.05) (width 0.08) (layer "F.Cu") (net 4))
 (segment (start 54.05 53.747394) (end 52.997394 54.8) (width 0.08) (layer "F.Cu") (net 4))
 (segment (start 51 55.3) (end 50.9 55.4) (width 0.08) (layer "F.Cu") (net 4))
 (segment (start 54.05 53.5) (end 54.05 53.747394) (width 0.08) (layer "F.Cu") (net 4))
 (segment (start 51 55) (end 51 55.3) (width 0.08) (layer "F.Cu") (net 4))
 (segment (start 51.2 54.8) (end 51 55) (width 0.08) (layer "F.Cu") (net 4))
 (segment (start 54.55 54.15) (end 55 54.6) (width 0.08) (layer "F.Cu") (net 3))
 (segment (start 57 55.4) (end 57 57.05) (width 0.08) (layer "F.Cu") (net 3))
 (segment (start 54.55 53.5) (end 54.55 54.15) (width 0.08) (layer "F.Cu") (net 3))
 (segment (start 55 54.6) (end 56.2 54.6) (width 0.08) (layer "F.Cu") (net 3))
 (segment (start 57 57.05) (end 56.65 57.4) (width 0.08) (layer "F.Cu") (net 3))
 (segment (start 56.2 54.6) (end 57 55.4) (width 0.08) (layer "F.Cu") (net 3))
 (segment (start 53 53) (end 53.55 53) (width 0.08) (layer "F.Cu") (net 1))
 (segment (start 52.9 52.9) (end 53 53) (width 0.08) (layer "F.Cu") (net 1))
 (segment (start 52.34 49.94) (end 52.9 50.5) (width 0.08) (layer "F.Cu") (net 1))
 (segment (start 52.9 50.5) (end 52.9 52.9) (width 0.08) (layer "F.Cu") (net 1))
 (segment (start 51.7 49.94) (end 52.34 49.94) (width 0.08) (layer "F.Cu") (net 1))
 (segment (start 53.6 52.05) (end 53.6 48) (width 0.08) (layer "F.Cu") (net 8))
 (segment (start 54.2 47.9) (end 54.25 47.85) (width 0.08) (layer "F.Cu") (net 8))
 (segment (start 53.6 48) (end 53.7 47.9) (width 0.08) (layer "F.Cu") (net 8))
 (segment (start 54.25 47.85) (end 54.25 46.8) (width 0.08) (layer "F.Cu") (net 8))
 (segment (start 54.05 52.5) (end 53.6 52.05) (width 0.08) (layer "F.Cu") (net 8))
 (segment (start 53.7 47.9) (end 54.2 47.9) (width 0.08) (layer "F.Cu") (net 8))
 (segment (start 53.25 52.2) (end 53.55 52.5) (width 0.08) (layer "F.Cu") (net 7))
 (segment (start 53.25 46.8) (end 53.25 52.2) (width 0.08) (layer "F.Cu") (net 7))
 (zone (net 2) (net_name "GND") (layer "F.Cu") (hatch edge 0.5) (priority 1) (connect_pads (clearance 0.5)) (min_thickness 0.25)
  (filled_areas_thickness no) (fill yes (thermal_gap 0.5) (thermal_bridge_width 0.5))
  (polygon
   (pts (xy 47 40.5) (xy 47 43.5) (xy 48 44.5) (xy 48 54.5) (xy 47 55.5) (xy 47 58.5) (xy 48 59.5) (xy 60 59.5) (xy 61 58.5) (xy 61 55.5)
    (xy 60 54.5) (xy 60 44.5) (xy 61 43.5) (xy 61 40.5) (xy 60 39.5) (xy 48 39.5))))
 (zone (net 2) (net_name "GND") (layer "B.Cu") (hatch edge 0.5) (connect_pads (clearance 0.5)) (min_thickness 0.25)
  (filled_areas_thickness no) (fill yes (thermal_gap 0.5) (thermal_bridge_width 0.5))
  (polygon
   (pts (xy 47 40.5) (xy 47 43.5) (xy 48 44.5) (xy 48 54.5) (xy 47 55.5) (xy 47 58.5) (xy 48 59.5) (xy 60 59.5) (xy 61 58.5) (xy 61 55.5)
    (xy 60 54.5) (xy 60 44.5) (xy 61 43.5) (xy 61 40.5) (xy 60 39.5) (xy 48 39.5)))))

